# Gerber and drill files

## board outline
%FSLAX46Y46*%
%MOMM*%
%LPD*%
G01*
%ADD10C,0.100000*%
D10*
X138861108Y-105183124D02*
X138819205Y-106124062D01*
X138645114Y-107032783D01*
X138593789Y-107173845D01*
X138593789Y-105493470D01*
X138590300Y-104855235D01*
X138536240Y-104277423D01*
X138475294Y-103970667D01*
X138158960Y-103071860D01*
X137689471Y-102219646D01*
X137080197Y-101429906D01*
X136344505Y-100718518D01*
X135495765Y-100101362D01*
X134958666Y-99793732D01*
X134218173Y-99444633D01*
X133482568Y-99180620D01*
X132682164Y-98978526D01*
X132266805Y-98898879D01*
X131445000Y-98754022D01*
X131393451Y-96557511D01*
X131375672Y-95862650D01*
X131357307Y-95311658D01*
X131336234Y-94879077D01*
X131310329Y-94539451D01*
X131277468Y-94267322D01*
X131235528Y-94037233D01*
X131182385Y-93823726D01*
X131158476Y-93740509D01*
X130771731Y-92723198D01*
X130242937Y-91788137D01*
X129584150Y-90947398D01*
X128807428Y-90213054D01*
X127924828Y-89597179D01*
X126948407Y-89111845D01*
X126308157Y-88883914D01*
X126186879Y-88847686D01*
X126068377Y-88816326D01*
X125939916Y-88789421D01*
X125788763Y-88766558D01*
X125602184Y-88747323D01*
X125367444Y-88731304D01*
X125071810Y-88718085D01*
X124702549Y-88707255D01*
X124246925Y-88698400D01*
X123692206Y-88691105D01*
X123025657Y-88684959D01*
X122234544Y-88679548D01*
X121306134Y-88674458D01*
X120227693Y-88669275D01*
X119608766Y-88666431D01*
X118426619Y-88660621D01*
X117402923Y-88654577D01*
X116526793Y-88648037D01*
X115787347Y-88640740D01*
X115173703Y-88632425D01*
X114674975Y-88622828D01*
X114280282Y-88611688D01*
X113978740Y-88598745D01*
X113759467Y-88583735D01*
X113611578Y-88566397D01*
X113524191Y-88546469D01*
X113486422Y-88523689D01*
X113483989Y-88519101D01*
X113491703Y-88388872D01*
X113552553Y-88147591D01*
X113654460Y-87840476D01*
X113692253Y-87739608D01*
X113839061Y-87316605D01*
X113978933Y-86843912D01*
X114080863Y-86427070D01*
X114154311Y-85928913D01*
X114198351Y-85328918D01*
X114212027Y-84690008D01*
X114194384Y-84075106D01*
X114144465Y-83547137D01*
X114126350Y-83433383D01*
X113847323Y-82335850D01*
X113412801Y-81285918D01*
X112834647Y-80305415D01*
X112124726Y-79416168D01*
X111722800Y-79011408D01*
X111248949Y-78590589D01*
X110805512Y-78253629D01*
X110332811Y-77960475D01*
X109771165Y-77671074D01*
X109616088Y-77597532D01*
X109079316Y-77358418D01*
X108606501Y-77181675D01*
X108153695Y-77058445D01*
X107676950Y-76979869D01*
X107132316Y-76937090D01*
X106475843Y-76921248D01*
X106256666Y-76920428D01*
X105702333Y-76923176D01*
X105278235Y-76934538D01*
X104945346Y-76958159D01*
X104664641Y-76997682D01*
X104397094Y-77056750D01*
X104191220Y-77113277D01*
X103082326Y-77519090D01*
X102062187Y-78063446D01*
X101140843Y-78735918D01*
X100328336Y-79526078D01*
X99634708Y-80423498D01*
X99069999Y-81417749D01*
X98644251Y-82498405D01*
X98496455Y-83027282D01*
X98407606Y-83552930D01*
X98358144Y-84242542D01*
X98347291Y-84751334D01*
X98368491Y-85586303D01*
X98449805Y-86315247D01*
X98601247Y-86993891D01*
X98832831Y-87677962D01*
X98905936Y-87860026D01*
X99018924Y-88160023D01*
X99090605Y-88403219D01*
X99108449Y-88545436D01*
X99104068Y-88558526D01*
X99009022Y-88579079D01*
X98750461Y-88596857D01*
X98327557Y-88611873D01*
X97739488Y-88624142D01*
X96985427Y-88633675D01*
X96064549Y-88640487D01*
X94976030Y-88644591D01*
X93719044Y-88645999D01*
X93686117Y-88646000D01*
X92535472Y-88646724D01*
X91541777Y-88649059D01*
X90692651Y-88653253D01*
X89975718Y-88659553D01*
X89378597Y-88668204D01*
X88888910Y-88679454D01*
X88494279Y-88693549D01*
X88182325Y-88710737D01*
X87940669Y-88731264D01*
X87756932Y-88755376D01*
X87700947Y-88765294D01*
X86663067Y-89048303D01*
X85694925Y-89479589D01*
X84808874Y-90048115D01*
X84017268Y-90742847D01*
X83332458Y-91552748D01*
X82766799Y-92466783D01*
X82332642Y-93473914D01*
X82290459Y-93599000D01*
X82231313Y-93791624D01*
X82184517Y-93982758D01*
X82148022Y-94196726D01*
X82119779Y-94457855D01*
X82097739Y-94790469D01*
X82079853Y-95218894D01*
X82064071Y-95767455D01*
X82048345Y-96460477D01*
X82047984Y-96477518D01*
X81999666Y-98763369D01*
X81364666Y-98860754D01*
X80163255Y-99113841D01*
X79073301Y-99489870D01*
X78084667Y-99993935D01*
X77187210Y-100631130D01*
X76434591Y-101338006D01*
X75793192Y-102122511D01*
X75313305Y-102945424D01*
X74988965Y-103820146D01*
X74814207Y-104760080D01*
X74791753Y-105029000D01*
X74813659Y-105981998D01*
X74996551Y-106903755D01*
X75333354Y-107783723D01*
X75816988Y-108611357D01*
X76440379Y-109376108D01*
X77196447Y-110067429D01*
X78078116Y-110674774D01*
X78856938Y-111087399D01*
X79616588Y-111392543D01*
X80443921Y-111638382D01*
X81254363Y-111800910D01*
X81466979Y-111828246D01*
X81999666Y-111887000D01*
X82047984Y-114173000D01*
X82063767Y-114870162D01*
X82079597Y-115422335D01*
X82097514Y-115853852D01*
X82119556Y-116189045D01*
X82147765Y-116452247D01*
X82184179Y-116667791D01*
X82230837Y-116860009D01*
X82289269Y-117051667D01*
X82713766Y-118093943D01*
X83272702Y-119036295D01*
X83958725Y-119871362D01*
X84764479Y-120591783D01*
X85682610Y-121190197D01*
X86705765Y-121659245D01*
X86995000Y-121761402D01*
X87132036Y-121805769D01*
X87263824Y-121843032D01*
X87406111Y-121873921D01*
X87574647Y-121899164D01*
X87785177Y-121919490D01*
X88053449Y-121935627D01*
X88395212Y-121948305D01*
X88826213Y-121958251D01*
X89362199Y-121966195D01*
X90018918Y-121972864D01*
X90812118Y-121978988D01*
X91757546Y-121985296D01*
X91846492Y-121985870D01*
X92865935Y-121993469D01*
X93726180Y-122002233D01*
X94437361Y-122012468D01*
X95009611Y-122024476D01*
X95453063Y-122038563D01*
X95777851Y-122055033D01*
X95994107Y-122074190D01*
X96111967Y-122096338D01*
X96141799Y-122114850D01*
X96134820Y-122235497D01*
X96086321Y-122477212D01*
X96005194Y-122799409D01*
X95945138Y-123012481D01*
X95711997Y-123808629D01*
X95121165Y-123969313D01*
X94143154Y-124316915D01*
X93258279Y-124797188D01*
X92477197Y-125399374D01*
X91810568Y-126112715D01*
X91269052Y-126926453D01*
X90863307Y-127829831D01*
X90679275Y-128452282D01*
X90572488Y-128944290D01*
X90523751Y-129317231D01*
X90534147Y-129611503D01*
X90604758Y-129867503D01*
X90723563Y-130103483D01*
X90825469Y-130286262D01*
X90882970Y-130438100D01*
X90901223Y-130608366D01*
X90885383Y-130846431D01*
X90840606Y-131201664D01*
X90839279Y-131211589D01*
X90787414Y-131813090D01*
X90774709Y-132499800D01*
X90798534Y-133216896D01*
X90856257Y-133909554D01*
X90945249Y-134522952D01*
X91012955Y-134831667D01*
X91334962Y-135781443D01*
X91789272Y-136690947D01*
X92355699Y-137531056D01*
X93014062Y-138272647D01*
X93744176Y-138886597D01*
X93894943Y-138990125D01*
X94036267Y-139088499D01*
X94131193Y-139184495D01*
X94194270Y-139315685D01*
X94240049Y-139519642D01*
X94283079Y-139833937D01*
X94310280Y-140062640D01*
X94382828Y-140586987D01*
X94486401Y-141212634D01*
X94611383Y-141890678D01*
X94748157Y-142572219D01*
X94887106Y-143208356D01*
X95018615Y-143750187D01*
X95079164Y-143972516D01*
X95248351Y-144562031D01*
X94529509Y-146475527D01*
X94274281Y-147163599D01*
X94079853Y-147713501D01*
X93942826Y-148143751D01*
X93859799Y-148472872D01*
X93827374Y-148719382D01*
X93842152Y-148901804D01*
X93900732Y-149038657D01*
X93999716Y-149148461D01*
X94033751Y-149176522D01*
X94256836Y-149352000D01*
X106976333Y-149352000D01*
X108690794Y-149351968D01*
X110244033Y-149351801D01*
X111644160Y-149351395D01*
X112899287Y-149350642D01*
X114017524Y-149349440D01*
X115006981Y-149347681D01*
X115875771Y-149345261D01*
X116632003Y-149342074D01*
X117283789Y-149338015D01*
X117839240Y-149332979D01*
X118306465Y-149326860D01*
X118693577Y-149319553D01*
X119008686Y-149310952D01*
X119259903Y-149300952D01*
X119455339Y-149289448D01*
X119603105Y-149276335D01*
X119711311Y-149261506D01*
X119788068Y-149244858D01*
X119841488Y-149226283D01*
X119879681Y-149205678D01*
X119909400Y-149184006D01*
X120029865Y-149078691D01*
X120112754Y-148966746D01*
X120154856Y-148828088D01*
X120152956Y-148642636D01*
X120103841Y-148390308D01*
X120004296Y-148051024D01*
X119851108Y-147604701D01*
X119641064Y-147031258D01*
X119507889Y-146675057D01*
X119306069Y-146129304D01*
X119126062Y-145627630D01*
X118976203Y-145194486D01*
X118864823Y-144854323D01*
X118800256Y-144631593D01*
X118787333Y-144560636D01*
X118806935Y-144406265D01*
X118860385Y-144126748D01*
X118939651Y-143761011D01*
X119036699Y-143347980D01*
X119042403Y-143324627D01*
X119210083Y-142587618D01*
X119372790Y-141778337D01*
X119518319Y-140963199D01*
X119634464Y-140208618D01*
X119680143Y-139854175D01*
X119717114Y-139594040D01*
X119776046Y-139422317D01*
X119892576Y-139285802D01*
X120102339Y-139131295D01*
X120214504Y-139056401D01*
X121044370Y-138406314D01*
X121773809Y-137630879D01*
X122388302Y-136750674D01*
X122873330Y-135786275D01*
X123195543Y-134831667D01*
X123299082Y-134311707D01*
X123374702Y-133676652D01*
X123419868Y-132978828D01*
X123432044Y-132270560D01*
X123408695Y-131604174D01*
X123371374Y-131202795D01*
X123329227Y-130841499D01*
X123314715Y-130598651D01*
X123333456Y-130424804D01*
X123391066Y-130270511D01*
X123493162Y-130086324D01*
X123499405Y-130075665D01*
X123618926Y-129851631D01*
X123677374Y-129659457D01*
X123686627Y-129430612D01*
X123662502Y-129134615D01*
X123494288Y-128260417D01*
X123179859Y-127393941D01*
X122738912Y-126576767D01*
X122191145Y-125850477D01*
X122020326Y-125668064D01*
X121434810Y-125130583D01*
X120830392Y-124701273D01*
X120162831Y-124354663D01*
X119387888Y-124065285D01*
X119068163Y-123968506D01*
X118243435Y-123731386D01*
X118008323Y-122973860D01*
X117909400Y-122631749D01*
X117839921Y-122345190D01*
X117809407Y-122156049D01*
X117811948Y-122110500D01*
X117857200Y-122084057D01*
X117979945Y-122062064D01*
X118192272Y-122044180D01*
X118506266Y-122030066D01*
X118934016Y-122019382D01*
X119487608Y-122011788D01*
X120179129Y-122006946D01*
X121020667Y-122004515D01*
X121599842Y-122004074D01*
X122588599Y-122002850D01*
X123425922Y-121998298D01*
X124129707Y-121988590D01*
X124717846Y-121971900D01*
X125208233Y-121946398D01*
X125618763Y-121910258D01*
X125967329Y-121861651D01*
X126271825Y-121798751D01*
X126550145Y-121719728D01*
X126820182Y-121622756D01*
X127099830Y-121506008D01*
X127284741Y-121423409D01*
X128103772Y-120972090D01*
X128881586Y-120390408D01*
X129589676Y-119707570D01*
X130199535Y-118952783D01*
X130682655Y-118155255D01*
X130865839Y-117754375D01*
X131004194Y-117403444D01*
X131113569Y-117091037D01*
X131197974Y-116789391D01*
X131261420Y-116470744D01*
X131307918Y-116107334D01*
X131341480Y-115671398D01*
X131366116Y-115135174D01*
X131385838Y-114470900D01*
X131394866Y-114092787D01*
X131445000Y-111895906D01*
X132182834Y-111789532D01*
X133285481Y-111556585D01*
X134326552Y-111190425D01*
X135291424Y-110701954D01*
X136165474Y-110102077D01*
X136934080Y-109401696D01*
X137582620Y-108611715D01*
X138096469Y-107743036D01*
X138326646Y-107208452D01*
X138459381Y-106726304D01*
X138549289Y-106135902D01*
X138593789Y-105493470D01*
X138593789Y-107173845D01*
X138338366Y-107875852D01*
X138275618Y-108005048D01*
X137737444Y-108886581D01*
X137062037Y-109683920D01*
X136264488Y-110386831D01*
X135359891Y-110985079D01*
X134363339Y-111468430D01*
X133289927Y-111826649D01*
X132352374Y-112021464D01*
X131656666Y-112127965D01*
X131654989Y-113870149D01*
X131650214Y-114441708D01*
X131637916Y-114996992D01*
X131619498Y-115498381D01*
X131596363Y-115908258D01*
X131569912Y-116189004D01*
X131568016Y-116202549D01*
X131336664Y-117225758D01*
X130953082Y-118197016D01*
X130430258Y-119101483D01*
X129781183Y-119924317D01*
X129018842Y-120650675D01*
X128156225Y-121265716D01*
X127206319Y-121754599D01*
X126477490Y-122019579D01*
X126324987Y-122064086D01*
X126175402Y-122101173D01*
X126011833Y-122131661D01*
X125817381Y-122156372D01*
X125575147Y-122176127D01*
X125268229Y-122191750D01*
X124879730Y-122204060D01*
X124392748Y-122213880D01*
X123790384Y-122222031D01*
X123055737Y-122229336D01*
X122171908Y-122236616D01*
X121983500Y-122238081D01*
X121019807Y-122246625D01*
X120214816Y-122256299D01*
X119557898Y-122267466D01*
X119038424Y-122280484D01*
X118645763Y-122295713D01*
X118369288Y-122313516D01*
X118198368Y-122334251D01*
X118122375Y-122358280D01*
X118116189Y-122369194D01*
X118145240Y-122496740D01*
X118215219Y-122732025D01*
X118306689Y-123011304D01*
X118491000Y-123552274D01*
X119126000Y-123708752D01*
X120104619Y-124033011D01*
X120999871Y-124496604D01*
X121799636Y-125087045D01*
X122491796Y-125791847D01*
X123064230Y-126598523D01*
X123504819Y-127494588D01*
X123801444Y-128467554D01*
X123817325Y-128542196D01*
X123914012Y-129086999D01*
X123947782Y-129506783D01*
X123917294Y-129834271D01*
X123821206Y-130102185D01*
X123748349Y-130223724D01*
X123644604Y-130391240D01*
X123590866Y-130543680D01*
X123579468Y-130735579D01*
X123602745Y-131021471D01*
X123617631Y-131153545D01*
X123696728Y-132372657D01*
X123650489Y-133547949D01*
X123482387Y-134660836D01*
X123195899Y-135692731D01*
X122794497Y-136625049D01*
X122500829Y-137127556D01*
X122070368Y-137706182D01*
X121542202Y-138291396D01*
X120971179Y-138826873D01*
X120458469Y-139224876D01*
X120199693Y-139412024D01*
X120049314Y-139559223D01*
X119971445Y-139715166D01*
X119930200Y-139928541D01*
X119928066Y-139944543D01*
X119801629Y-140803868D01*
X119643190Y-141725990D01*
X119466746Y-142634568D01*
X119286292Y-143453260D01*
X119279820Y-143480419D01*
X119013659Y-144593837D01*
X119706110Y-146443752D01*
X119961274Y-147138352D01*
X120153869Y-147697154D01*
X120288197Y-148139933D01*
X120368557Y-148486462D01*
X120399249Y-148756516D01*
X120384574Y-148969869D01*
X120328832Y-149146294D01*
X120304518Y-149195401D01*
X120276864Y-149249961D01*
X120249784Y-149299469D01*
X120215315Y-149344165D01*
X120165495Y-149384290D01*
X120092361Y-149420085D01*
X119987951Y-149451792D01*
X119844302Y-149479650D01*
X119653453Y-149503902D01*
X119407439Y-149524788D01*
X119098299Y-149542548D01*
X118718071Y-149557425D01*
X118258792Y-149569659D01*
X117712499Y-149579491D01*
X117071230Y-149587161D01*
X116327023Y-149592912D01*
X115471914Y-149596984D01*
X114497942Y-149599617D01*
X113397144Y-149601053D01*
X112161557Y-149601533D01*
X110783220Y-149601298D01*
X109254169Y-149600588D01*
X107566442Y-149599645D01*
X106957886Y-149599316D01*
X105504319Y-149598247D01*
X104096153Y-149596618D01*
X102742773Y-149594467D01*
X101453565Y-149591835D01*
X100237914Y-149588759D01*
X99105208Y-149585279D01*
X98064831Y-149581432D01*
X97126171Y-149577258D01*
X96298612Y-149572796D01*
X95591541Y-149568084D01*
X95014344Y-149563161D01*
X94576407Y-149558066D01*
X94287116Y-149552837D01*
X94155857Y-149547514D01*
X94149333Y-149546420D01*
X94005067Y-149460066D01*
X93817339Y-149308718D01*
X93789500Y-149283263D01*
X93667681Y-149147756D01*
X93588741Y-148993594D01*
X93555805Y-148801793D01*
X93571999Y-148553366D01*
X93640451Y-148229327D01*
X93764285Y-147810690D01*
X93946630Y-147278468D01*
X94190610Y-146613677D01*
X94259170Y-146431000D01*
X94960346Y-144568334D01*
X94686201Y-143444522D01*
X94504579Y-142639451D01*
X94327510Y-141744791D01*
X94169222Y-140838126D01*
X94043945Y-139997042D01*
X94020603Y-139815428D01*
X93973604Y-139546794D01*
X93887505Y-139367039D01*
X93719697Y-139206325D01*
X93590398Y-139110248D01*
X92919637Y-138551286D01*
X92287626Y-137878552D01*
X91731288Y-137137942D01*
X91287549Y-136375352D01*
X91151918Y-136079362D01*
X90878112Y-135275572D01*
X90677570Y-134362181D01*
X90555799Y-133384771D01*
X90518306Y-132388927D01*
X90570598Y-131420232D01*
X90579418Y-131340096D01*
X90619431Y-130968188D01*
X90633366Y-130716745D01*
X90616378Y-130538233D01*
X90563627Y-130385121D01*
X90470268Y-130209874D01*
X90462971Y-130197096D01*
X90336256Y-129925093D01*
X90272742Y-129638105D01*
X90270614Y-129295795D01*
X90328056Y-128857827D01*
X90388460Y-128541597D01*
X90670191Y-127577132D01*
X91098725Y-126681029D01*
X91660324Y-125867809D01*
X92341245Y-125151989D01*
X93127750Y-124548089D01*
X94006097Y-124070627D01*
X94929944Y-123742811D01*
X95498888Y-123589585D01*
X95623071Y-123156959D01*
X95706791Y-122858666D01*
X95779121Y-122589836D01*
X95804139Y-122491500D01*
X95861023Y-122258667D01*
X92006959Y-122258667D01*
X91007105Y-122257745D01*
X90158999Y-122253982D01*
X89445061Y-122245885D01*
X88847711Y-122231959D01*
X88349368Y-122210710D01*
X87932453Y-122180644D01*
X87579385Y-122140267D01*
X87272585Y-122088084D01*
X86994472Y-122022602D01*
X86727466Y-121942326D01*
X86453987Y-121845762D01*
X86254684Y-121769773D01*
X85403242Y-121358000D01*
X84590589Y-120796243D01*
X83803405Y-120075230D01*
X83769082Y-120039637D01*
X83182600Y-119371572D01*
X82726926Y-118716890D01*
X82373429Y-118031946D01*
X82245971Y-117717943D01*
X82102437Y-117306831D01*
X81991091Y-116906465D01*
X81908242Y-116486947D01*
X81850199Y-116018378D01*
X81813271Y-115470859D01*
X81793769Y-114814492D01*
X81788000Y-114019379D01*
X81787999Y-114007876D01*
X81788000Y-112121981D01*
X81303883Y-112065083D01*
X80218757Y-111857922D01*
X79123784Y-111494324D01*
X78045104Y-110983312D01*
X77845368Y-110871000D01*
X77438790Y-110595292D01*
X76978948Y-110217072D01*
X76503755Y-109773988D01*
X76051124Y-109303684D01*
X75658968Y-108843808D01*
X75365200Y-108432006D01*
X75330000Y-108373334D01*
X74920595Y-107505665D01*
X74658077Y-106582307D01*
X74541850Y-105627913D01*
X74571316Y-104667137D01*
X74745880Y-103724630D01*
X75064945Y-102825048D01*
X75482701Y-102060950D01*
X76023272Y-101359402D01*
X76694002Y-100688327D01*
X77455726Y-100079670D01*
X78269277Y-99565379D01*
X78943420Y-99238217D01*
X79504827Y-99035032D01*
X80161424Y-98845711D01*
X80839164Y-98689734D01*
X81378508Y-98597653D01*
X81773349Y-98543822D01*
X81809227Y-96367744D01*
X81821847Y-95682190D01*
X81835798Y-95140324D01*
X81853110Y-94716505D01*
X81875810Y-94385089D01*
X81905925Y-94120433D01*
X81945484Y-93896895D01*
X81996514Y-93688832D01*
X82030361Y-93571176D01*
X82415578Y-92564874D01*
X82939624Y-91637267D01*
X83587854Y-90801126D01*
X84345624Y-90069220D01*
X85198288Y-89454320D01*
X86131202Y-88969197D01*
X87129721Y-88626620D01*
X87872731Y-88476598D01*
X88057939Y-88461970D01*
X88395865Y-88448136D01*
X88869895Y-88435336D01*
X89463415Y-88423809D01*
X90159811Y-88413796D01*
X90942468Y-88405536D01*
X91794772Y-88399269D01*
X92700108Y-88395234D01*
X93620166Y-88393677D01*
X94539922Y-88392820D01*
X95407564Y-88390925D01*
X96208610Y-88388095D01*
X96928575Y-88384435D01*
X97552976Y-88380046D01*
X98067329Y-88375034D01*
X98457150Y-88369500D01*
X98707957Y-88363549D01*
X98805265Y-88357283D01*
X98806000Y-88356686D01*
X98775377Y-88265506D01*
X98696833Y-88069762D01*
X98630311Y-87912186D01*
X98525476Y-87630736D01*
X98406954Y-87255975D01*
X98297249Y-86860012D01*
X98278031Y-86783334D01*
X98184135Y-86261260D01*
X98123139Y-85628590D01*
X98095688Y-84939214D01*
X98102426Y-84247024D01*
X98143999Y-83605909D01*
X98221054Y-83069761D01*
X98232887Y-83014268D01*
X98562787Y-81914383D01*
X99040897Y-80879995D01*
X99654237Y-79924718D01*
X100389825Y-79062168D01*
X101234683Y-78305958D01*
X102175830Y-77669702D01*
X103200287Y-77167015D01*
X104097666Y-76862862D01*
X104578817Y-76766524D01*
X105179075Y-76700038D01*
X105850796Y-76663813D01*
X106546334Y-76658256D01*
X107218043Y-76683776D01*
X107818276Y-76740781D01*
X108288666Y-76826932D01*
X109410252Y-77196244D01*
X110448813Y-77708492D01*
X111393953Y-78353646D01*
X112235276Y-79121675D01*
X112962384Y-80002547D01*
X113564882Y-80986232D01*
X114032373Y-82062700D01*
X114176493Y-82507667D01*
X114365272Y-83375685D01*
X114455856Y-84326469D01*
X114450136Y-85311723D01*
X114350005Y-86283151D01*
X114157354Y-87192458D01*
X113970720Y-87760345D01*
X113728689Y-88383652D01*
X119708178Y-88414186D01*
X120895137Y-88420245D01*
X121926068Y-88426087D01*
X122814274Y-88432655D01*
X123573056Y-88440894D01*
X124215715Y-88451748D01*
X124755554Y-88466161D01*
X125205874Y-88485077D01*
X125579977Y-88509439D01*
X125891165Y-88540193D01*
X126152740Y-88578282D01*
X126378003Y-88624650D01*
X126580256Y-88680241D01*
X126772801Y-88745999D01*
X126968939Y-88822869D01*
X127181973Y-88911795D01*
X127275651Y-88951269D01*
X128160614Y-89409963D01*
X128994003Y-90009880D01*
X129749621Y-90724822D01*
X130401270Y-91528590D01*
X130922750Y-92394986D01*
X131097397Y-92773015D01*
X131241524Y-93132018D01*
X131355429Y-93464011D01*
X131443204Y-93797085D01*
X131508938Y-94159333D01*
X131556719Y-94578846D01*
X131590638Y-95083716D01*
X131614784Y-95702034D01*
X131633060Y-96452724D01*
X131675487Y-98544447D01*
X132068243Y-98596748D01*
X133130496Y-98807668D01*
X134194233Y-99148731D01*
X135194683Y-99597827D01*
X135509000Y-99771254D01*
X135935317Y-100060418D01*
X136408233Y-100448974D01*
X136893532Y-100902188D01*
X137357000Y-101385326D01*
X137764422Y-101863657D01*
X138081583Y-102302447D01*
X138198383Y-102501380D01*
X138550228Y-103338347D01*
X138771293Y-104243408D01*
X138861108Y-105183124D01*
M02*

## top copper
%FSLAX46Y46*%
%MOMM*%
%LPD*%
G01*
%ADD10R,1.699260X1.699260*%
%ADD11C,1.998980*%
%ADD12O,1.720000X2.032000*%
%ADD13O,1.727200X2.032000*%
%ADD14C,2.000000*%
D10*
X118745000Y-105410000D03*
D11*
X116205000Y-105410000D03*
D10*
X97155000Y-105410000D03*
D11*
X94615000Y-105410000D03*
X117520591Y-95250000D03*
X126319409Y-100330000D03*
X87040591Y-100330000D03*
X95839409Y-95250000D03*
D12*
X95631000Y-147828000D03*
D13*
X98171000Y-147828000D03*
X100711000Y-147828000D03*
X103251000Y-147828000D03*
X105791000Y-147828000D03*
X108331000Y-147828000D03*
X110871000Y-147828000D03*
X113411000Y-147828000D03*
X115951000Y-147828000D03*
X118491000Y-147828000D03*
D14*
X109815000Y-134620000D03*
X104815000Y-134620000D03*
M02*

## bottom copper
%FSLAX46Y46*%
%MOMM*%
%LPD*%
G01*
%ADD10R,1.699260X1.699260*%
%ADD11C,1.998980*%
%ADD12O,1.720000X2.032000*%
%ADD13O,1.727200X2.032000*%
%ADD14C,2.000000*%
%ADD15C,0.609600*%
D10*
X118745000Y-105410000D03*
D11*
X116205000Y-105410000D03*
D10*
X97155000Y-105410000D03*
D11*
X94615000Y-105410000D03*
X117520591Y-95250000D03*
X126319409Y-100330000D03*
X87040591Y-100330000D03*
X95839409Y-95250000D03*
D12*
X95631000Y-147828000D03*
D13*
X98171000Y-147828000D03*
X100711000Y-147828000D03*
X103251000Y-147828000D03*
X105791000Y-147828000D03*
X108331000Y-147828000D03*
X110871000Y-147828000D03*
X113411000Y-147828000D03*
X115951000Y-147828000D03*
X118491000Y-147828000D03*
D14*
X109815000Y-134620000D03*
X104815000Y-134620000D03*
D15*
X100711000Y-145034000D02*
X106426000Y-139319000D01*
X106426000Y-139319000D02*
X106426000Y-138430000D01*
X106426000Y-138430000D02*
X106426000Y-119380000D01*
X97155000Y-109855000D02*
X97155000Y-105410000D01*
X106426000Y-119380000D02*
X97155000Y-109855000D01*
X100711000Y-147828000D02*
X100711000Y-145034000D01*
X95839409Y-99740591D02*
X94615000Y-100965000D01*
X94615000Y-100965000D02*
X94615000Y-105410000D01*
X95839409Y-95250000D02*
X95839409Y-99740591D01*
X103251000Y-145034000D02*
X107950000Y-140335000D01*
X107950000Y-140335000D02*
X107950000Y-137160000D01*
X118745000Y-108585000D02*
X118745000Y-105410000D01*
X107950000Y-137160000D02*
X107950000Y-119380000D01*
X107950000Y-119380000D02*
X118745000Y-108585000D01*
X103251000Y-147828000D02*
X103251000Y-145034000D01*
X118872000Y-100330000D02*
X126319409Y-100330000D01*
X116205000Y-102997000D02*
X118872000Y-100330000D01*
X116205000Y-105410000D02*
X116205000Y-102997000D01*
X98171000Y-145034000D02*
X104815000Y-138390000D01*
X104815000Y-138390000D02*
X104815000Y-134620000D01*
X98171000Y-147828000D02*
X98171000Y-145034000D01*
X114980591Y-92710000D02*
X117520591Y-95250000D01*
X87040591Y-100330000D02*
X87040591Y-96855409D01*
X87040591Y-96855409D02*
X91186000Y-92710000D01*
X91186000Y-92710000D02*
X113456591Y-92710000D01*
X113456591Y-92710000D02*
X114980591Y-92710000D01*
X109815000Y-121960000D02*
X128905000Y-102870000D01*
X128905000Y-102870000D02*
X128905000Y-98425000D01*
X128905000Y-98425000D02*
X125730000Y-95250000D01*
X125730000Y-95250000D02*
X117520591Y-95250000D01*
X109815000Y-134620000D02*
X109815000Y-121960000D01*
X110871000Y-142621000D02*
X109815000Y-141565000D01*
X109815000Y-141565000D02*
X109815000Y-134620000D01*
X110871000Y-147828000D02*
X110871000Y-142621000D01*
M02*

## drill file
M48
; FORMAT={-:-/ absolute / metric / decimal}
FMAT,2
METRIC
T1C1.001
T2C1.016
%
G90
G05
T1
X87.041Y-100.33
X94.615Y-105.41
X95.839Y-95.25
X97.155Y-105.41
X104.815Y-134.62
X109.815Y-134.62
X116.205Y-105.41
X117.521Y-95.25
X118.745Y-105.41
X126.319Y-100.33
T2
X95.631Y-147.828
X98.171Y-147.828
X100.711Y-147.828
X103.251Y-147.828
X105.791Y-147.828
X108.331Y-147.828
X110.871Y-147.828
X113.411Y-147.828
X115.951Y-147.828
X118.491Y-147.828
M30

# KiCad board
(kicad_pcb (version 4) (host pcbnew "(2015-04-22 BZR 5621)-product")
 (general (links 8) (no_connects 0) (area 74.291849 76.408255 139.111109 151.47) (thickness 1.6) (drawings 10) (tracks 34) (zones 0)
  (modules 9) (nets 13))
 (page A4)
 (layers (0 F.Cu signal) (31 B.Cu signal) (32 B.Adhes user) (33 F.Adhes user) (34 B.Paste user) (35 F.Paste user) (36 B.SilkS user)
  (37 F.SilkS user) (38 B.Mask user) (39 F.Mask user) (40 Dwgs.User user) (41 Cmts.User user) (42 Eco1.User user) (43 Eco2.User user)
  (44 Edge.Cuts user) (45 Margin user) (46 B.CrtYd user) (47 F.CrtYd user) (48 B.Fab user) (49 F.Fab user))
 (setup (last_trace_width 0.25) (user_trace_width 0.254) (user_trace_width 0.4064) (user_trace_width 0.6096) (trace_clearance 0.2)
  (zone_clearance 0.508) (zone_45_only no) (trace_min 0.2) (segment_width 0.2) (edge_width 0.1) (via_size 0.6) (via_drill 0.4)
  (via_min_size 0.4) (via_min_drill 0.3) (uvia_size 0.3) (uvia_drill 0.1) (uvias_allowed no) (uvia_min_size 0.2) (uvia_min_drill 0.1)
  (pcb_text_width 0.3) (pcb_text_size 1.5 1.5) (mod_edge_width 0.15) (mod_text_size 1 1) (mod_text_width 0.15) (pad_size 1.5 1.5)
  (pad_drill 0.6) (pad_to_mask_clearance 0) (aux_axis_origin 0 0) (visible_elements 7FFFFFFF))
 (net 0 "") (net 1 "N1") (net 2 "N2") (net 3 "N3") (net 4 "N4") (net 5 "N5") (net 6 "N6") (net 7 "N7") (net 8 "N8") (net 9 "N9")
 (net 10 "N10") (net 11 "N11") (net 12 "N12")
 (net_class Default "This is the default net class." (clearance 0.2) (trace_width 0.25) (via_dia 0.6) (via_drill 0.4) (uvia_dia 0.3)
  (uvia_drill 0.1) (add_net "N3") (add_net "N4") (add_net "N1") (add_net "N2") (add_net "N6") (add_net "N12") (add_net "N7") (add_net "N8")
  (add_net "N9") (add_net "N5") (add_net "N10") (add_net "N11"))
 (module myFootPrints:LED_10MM (layer F.Cu) (at 117.475 105.41 180)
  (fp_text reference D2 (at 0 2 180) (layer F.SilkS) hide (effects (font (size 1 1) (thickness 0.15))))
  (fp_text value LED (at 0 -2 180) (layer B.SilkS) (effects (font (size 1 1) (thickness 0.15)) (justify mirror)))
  (pad 1 thru_hole rect (at -1.27 0 270) (size 1.69926 1.69926) (drill 1.00076) (layers *.Cu *.Mask F.SilkS) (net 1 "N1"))
  (pad 2 thru_hole circle (at 1.27 0 180) (size 1.99898 1.99898) (drill 1.00076) (layers *.Cu *.Mask F.SilkS) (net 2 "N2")))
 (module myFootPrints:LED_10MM (layer F.Cu) (at 95.885 105.41 180)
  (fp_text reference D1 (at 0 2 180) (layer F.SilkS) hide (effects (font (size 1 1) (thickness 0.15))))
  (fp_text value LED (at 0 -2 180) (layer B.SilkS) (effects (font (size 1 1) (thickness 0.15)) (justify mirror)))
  (pad 1 thru_hole rect (at -1.27 0 270) (size 1.69926 1.69926) (drill 1.00076) (layers *.Cu *.Mask F.SilkS) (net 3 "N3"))
  (pad 2 thru_hole circle (at 1.27 0 180) (size 1.99898 1.99898) (drill 1.00076) (layers *.Cu *.Mask F.SilkS) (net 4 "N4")))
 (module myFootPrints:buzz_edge (layer F.Cu) (at 106.68 113.03)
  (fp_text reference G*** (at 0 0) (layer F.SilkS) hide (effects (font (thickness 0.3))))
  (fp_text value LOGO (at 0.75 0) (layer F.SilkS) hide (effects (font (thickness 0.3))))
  (fp_poly
   (pts (xy 32.181108 -7.846876) (xy 32.139205 -6.905938) (xy 31.965114 -5.997217) (xy 31.913789 -5.856155) (xy 31.913789 -7.53653)
    (xy 31.9103 -8.174765) (xy 31.85624 -8.752577) (xy 31.795294 -9.059333) (xy 31.47896 -9.95814) (xy 31.009471 -10.810354)
    (xy 30.400197 -11.600094) (xy 29.664505 -12.311482) (xy 28.815765 -12.928638) (xy 28.278666 -13.236268) (xy 27.538173 -13.585367)
    (xy 26.802568 -13.84938) (xy 26.002164 -14.051474) (xy 25.586805 -14.131121) (xy 24.765 -14.275978) (xy 24.713451 -16.472489)
    (xy 24.695672 -17.16735) (xy 24.677307 -17.718342) (xy 24.656234 -18.150923) (xy 24.630329 -18.490549) (xy 24.597468 -18.762678)
    (xy 24.555528 -18.992767) (xy 24.502385 -19.206274) (xy 24.478476 -19.289491) (xy 24.091731 -20.306802) (xy 23.562937 -21.241863)
    (xy 22.90415 -22.082602) (xy 22.127428 -22.816946) (xy 21.244828 -23.432821) (xy 20.268407 -23.918155) (xy 19.628157 -24.146086)
    (xy 19.506879 -24.182314) (xy 19.388377 -24.213674) (xy 19.259916 -24.240579) (xy 19.108763 -24.263442) (xy 18.922184 -24.282677)
    (xy 18.687444 -24.298696) (xy 18.39181 -24.311915) (xy 18.022549 -24.322745) (xy 17.566925 -24.3316) (xy 17.012206 -24.338895)
    (xy 16.345657 -24.345041) (xy 15.554544 -24.350452) (xy 14.626134 -24.355542) (xy 13.547693 -24.360725) (xy 12.928766 -24.363569)
    (xy 11.746619 -24.369379) (xy 10.722923 -24.375423) (xy 9.846793 -24.381963) (xy 9.107347 -24.38926) (xy 8.493703 -24.397575)
    (xy 7.994975 -24.407172) (xy 7.600282 -24.418312) (xy 7.29874 -24.431255) (xy 7.079467 -24.446265) (xy 6.931578 -24.463603)
    (xy 6.844191 -24.483531) (xy 6.806422 -24.506311) (xy 6.803989 -24.510899) (xy 6.811703 -24.641128) (xy 6.872553 -24.882409)
    (xy 6.97446 -25.189524) (xy 7.012253 -25.290392) (xy 7.159061 -25.713395) (xy 7.298933 -26.186088) (xy 7.400863 -26.60293)
    (xy 7.474311 -27.101087) (xy 7.518351 -27.701082) (xy 7.532027 -28.339992) (xy 7.514384 -28.954894) (xy 7.464465 -29.482863)
    (xy 7.44635 -29.596617) (xy 7.167323 -30.69415) (xy 6.732801 -31.744082) (xy 6.154647 -32.724585) (xy 5.444726 -33.613832)
    (xy 5.0428 -34.018592) (xy 4.568949 -34.439411) (xy 4.125512 -34.776371) (xy 3.652811 -35.069525) (xy 3.091165 -35.358926)
    (xy 2.936088 -35.432468) (xy 2.399316 -35.671582) (xy 1.926501 -35.848325) (xy 1.473695 -35.971555) (xy 0.99695 -36.050131)
    (xy 0.452316 -36.09291) (xy -0.204157 -36.108752) (xy -0.423334 -36.109572) (xy -0.977667 -36.106824) (xy -1.401765 -36.095462)
    (xy -1.734654 -36.071841) (xy -2.015359 -36.032318) (xy -2.282906 -35.97325) (xy -2.48878 -35.916723) (xy -3.597674 -35.51091)
    (xy -4.617813 -34.966554) (xy -5.539157 -34.294082) (xy -6.351664 -33.503922) (xy -7.045292 -32.606502) (xy -7.610001 -31.612251)
    (xy -8.035749 -30.531595) (xy -8.183545 -30.002718) (xy -8.272394 -29.47707) (xy -8.321856 -28.787458) (xy -8.332709 -28.278666)
    (xy -8.311509 -27.443697) (xy -8.230195 -26.714753) (xy -8.078753 -26.036109) (xy -7.847169 -25.352038) (xy -7.774064 -25.169974)
    (xy -7.661076 -24.869977) (xy -7.589395 -24.626781) (xy -7.571551 -24.484564) (xy -7.575932 -24.471474) (xy -7.670978 -24.450921)
    (xy -7.929539 -24.433143) (xy -8.352443 -24.418127) (xy -8.940512 -24.405858) (xy -9.694573 -24.396325) (xy -10.615451 -24.389513)
    (xy -11.70397 -24.385409) (xy -12.960956 -24.384001) (xy -12.993883 -24.384) (xy -14.144528 -24.383276) (xy -15.138223 -24.380941)
    (xy -15.987349 -24.376747) (xy -16.704282 -24.370447) (xy -17.301403 -24.361796) (xy -17.79109 -24.350546) (xy -18.185721 -24.336451)
    (xy -18.497675 -24.319263) (xy -18.739331 -24.298736) (xy -18.923068 -24.274624) (xy -18.979053 -24.264706) (xy -20.016933 -23.981697)
    (xy -20.985075 -23.550411) (xy -21.871126 -22.981885) (xy -22.662732 -22.287153) (xy -23.347542 -21.477252) (xy -23.913201 -20.563217)
    (xy -24.347358 -19.556086) (xy -24.389541 -19.431) (xy -24.448687 -19.238376) (xy -24.495483 -19.047242) (xy -24.531978 -18.833274)
    (xy -24.560221 -18.572145) (xy -24.582261 -18.239531) (xy -24.600147 -17.811106) (xy -24.615929 -17.262545) (xy -24.631655 -16.569523)
    (xy -24.632016 -16.552482) (xy -24.680334 -14.266631) (xy -25.315334 -14.169246) (xy -26.516745 -13.916159) (xy -27.606699 -13.54013)
    (xy -28.595333 -13.036065) (xy -29.49279 -12.39887) (xy -30.245409 -11.691994) (xy -30.886808 -10.907489) (xy -31.366695 -10.084576)
    (xy -31.691035 -9.209854) (xy -31.865793 -8.26992) (xy -31.888247 -8.001) (xy -31.866341 -7.048002) (xy -31.683449 -6.126245)
    (xy -31.346646 -5.246277) (xy -30.863012 -4.418643) (xy -30.239621 -3.653892) (xy -29.483553 -2.962571) (xy -28.601884 -2.355226)
    (xy -27.823062 -1.942601) (xy -27.063412 -1.637457) (xy -26.236079 -1.391618) (xy -25.425637 -1.22909) (xy -25.213021 -1.201754)
    (xy -24.680334 -1.143) (xy -24.632016 1.143) (xy -24.616233 1.840162) (xy -24.600403 2.392335) (xy -24.582486 2.823852)
    (xy -24.560444 3.159045) (xy -24.532235 3.422247) (xy -24.495821 3.637791) (xy -24.449163 3.830009) (xy -24.390731 4.021667)
    (xy -23.966234 5.063943) (xy -23.407298 6.006295) (xy -22.721275 6.841362) (xy -21.915521 7.561783) (xy -20.99739 8.160197)
    (xy -19.974235 8.629245) (xy -19.685 8.731402) (xy -19.547964 8.775769) (xy -19.416176 8.813032) (xy -19.273889 8.843921)
    (xy -19.105353 8.869164) (xy -18.894823 8.88949) (xy -18.626551 8.905627) (xy -18.284788 8.918305) (xy -17.853787 8.928251)
    (xy -17.317801 8.936195) (xy -16.661082 8.942864) (xy -15.867882 8.948988) (xy -14.922454 8.955296) (xy -14.833508 8.95587)
    (xy -13.814065 8.963469) (xy -12.95382 8.972233) (xy -12.242639 8.982468) (xy -11.670389 8.994476) (xy -11.226937 9.008563)
    (xy -10.902149 9.025033) (xy -10.685893 9.04419) (xy -10.568033 9.066338) (xy -10.538201 9.08485) (xy -10.54518 9.205497)
    (xy -10.593679 9.447212) (xy -10.674806 9.769409) (xy -10.734862 9.982481) (xy -10.968003 10.778629) (xy -11.558835 10.939313)
    (xy -12.536846 11.286915) (xy -13.421721 11.767188) (xy -14.202803 12.369374) (xy -14.869432 13.082715) (xy -15.410948 13.896453)
    (xy -15.816693 14.799831) (xy -16.000725 15.422282) (xy -16.107512 15.91429) (xy -16.156249 16.287231) (xy -16.145853 16.581503)
    (xy -16.075242 16.837503) (xy -15.956437 17.073483) (xy -15.854531 17.256262) (xy -15.79703 17.4081) (xy -15.778777 17.578366)
    (xy -15.794617 17.816431) (xy -15.839394 18.171664) (xy -15.840721 18.181589) (xy -15.892586 18.78309) (xy -15.905291 19.4698)
    (xy -15.881466 20.186896) (xy -15.823743 20.879554) (xy -15.734751 21.492952) (xy -15.667045 21.801667) (xy -15.345038 22.751443)
    (xy -14.890728 23.660947) (xy -14.324301 24.501056) (xy -13.665938 25.242647) (xy -12.935824 25.856597) (xy -12.785057 25.960125)
    (xy -12.643733 26.058499) (xy -12.548807 26.154495) (xy -12.48573 26.285685) (xy -12.439951 26.489642) (xy -12.396921 26.803937)
    (xy -12.36972 27.03264) (xy -12.297172 27.556987) (xy -12.193599 28.182634) (xy -12.068617 28.860678) (xy -11.931843 29.542219)
    (xy -11.792894 30.178356) (xy -11.661385 30.720187) (xy -11.600836 30.942516) (xy -11.431649 31.532031) (xy -12.150491 33.445527)
    (xy -12.405719 34.133599) (xy -12.600147 34.683501) (xy -12.737174 35.113751) (xy -12.820201 35.442872) (xy -12.852626 35.689382)
    (xy -12.837848 35.871804) (xy -12.779268 36.008657) (xy -12.680284 36.118461) (xy -12.646249 36.146522) (xy -12.423164 36.322)
    (xy 0.296333 36.322) (xy 2.010794 36.321968) (xy 3.564033 36.321801) (xy 4.96416 36.321395) (xy 6.219287 36.320642)
    (xy 7.337524 36.31944) (xy 8.326981 36.317681) (xy 9.195771 36.315261) (xy 9.952003 36.312074) (xy 10.603789 36.308015)
    (xy 11.15924 36.302979) (xy 11.626465 36.29686) (xy 12.013577 36.289553) (xy 12.328686 36.280952) (xy 12.579903 36.270952)
    (xy 12.775339 36.259448) (xy 12.923105 36.246335) (xy 13.031311 36.231506) (xy 13.108068 36.214858) (xy 13.161488 36.196283)
    (xy 13.199681 36.175678) (xy 13.2294 36.154006) (xy 13.349865 36.048691) (xy 13.432754 35.936746) (xy 13.474856 35.798088)
    (xy 13.472956 35.612636) (xy 13.423841 35.360308) (xy 13.324296 35.021024) (xy 13.171108 34.574701) (xy 12.961064 34.001258)
    (xy 12.827889 33.645057) (xy 12.626069 33.099304) (xy 12.446062 32.59763) (xy 12.296203 32.164486) (xy 12.184823 31.824323)
    (xy 12.120256 31.601593) (xy 12.107333 31.530636) (xy 12.126935 31.376265) (xy 12.180385 31.096748) (xy 12.259651 30.731011)
    (xy 12.356699 30.31798) (xy 12.362403 30.294627) (xy 12.530083 29.557618) (xy 12.69279 28.748337) (xy 12.838319 27.933199)
    (xy 12.954464 27.178618) (xy 13.000143 26.824175) (xy 13.037114 26.56404) (xy 13.096046 26.392317) (xy 13.212576 26.255802)
    (xy 13.422339 26.101295) (xy 13.534504 26.026401) (xy 14.36437 25.376314) (xy 15.093809 24.600879) (xy 15.708302 23.720674)
    (xy 16.19333 22.756275) (xy 16.515543 21.801667) (xy 16.619082 21.281707) (xy 16.694702 20.646652) (xy 16.739868 19.948828)
    (xy 16.752044 19.24056) (xy 16.728695 18.574174) (xy 16.691374 18.172795) (xy 16.649227 17.811499) (xy 16.634715 17.568651)
    (xy 16.653456 17.394804) (xy 16.711066 17.240511) (xy 16.813162 17.056324) (xy 16.819405 17.045665) (xy 16.938926 16.821631)
    (xy 16.997374 16.629457) (xy 17.006627 16.400612) (xy 16.982502 16.104615) (xy 16.814288 15.230417) (xy 16.499859 14.363941)
    (xy 16.058912 13.546767) (xy 15.511145 12.820477) (xy 15.340326 12.638064) (xy 14.75481 12.100583) (xy 14.150392 11.671273)
    (xy 13.482831 11.324663) (xy 12.707888 11.035285) (xy 12.388163 10.938506) (xy 11.563435 10.701386) (xy 11.328323 9.94386)
    (xy 11.2294 9.601749) (xy 11.159921 9.31519) (xy 11.129407 9.126049) (xy 11.131948 9.0805) (xy 11.1772 9.054057) (xy 11.299945 9.032064)
    (xy 11.512272 9.01418) (xy 11.826266 9.000066) (xy 12.254016 8.989382) (xy 12.807608 8.981788) (xy 13.499129 8.976946)
    (xy 14.340667 8.974515) (xy 14.919842 8.974074) (xy 15.908599 8.97285) (xy 16.745922 8.968298) (xy 17.449707 8.95859)
    (xy 18.037846 8.9419) (xy 18.528233 8.916398) (xy 18.938763 8.880258) (xy 19.287329 8.831651) (xy 19.591825 8.768751)
    (xy 19.870145 8.689728) (xy 20.140182 8.592756) (xy 20.41983 8.476008) (xy 20.604741 8.393409) (xy 21.423772 7.94209)
    (xy 22.201586 7.360408) (xy 22.909676 6.67757) (xy 23.519535 5.922783) (xy 24.002655 5.125255) (xy 24.185839 4.724375)
    (xy 24.324194 4.373444) (xy 24.433569 4.061037) (xy 24.517974 3.759391) (xy 24.58142 3.440744) (xy 24.627918 3.077334)
    (xy 24.66148 2.641398) (xy 24.686116 2.105174) (xy 24.705838 1.4409) (xy 24.714866 1.062787) (xy 24.765 -1.134094)
    (xy 25.502834 -1.240468) (xy 26.605481 -1.473415) (xy 27.646552 -1.839575) (xy 28.611424 -2.328046) (xy 29.485474 -2.927923)
    (xy 30.25408 -3.628304) (xy 30.90262 -4.418285) (xy 31.416469 -5.286964) (xy 31.646646 -5.821548) (xy 31.779381 -6.303696)
    (xy 31.869289 -6.894098) (xy 31.913789 -7.53653) (xy 31.913789 -5.856155) (xy 31.658366 -5.154148) (xy 31.595618 -5.024952)
    (xy 31.057444 -4.143419) (xy 30.382037 -3.34608) (xy 29.584488 -2.643169) (xy 28.679891 -2.044921) (xy 27.683339 -1.56157)
    (xy 26.609927 -1.203351) (xy 25.672374 -1.008536) (xy 24.976666 -0.902035) (xy 24.974989 0.840149) (xy 24.970214 1.411708)
    (xy 24.957916 1.966992) (xy 24.939498 2.468381) (xy 24.916363 2.878258) (xy 24.889912 3.159004) (xy 24.888016 3.172549)
    (xy 24.656664 4.195758) (xy 24.273082 5.167016) (xy 23.750258 6.071483) (xy 23.101183 6.894317) (xy 22.338842 7.620675)
    (xy 21.476225 8.235716) (xy 20.526319 8.724599) (xy 19.79749 8.989579) (xy 19.644987 9.034086) (xy 19.495402 9.071173)
    (xy 19.331833 9.101661) (xy 19.137381 9.126372) (xy 18.895147 9.146127) (xy 18.588229 9.16175) (xy 18.19973 9.17406)
    (xy 17.712748 9.18388) (xy 17.110384 9.192031) (xy 16.375737 9.199336) (xy 15.491908 9.206616) (xy 15.3035 9.208081)
    (xy 14.339807 9.216625) (xy 13.534816 9.226299) (xy 12.877898 9.237466) (xy 12.358424 9.250484) (xy 11.965763 9.265713)
    (xy 11.689288 9.283516) (xy 11.518368 9.304251) (xy 11.442375 9.32828) (xy 11.436189 9.339194) (xy 11.46524 9.46674)
    (xy 11.535219 9.702025) (xy 11.626689 9.981304) (xy 11.811 10.522274) (xy 12.446 10.678752) (xy 13.424619 11.003011)
    (xy 14.319871 11.466604) (xy 15.119636 12.057045) (xy 15.811796 12.761847) (xy 16.38423 13.568523) (xy 16.824819 14.464588)
    (xy 17.121444 15.437554) (xy 17.137325 15.512196) (xy 17.234012 16.056999) (xy 17.267782 16.476783) (xy 17.237294 16.804271)
    (xy 17.141206 17.072185) (xy 17.068349 17.193724) (xy 16.964604 17.36124) (xy 16.910866 17.51368) (xy 16.899468 17.705579)
    (xy 16.922745 17.991471) (xy 16.937631 18.123545) (xy 17.016728 19.342657) (xy 16.970489 20.517949) (xy 16.802387 21.630836)
    (xy 16.515899 22.662731) (xy 16.114497 23.595049) (xy 15.820829 24.097556) (xy 15.390368 24.676182) (xy 14.862202 25.261396)
    (xy 14.291179 25.796873) (xy 13.778469 26.194876) (xy 13.519693 26.382024) (xy 13.369314 26.529223) (xy 13.291445 26.685166)
    (xy 13.2502 26.898541) (xy 13.248066 26.914543) (xy 13.121629 27.773868) (xy 12.96319 28.69599) (xy 12.786746 29.604568)
    (xy 12.606292 30.42326) (xy 12.59982 30.450419) (xy 12.333659 31.563837) (xy 13.02611 33.413752) (xy 13.281274 34.108352)
    (xy 13.473869 34.667154) (xy 13.608197 35.109933) (xy 13.688557 35.456462) (xy 13.719249 35.726516) (xy 13.704574 35.939869)
    (xy 13.648832 36.116294) (xy 13.624518 36.165401) (xy 13.596864 36.219961) (xy 13.569784 36.269469) (xy 13.535315 36.314165)
    (xy 13.485495 36.35429) (xy 13.412361 36.390085) (xy 13.307951 36.421792) (xy 13.164302 36.44965) (xy 12.973453 36.473902)
    (xy 12.727439 36.494788) (xy 12.418299 36.512548) (xy 12.038071 36.527425) (xy 11.578792 36.539659) (xy 11.032499 36.549491)
    (xy 10.39123 36.557161) (xy 9.647023 36.562912) (xy 8.791914 36.566984) (xy 7.817942 36.569617) (xy 6.717144 36.571053)
    (xy 5.481557 36.571533) (xy 4.10322 36.571298) (xy 2.574169 36.570588) (xy 0.886442 36.569645) (xy 0.277886 36.569316)
    (xy -1.175681 36.568247) (xy -2.583847 36.566618) (xy -3.937227 36.564467) (xy -5.226435 36.561835) (xy -6.442086 36.558759)
    (xy -7.574792 36.555279) (xy -8.615169 36.551432) (xy -9.553829 36.547258) (xy -10.381388 36.542796) (xy -11.088459 36.538084)
    (xy -11.665656 36.533161) (xy -12.103593 36.528066) (xy -12.392884 36.522837) (xy -12.524143 36.517514) (xy -12.530667 36.51642)
    (xy -12.674933 36.430066) (xy -12.862661 36.278718) (xy -12.8905 36.253263) (xy -13.012319 36.117756) (xy -13.091259 35.963594)
    (xy -13.124195 35.771793) (xy -13.108001 35.523366) (xy -13.039549 35.199327) (xy -12.915715 34.78069) (xy -12.73337 34.248468)
    (xy -12.48939 33.583677) (xy -12.42083 33.401) (xy -11.719654 31.538334) (xy -11.993799 30.414522) (xy -12.175421 29.609451)
    (xy -12.35249 28.714791) (xy -12.510778 27.808126) (xy -12.636055 26.967042) (xy -12.659397 26.785428) (xy -12.706396 26.516794)
    (xy -12.792495 26.337039) (xy -12.960303 26.176325) (xy -13.089602 26.080248) (xy -13.760363 25.521286) (xy -14.392374 24.848552)
    (xy -14.948712 24.107942) (xy -15.392451 23.345352) (xy -15.528082 23.049362) (xy -15.801888 22.245572) (xy -16.00243 21.332181)
    (xy -16.124201 20.354771) (xy -16.161694 19.358927) (xy -16.109402 18.390232) (xy -16.100582 18.310096) (xy -16.060569 17.938188)
    (xy -16.046634 17.686745) (xy -16.063622 17.508233) (xy -16.116373 17.355121) (xy -16.209732 17.179874) (xy -16.217029 17.167096)
    (xy -16.343744 16.895093) (xy -16.407258 16.608105) (xy -16.409386 16.265795) (xy -16.351944 15.827827) (xy -16.29154 15.511597)
    (xy -16.009809 14.547132) (xy -15.581275 13.651029) (xy -15.019676 12.837809) (xy -14.338755 12.121989) (xy -13.55225 11.518089)
    (xy -12.673903 11.040627) (xy -11.750056 10.712811) (xy -11.181112 10.559585) (xy -11.056929 10.126959) (xy -10.973209 9.828666)
    (xy -10.900879 9.559836) (xy -10.875861 9.4615) (xy -10.818977 9.228667) (xy -14.673041 9.228667) (xy -15.672895 9.227745)
    (xy -16.521001 9.223982) (xy -17.234939 9.215885) (xy -17.832289 9.201959) (xy -18.330632 9.18071) (xy -18.747547 9.150644)
    (xy -19.100615 9.110267) (xy -19.407415 9.058084) (xy -19.685528 8.992602) (xy -19.952534 8.912326) (xy -20.226013 8.815762)
    (xy -20.425316 8.739773) (xy -21.276758 8.328) (xy -22.089411 7.766243) (xy -22.876595 7.04523) (xy -22.910918 7.009637)
    (xy -23.4974 6.341572) (xy -23.953074 5.68689) (xy -24.306571 5.001946) (xy -24.434029 4.687943) (xy -24.577563 4.276831)
    (xy -24.688909 3.876465) (xy -24.771758 3.456947) (xy -24.829801 2.988378) (xy -24.866729 2.440859) (xy -24.886231 1.784492)
    (xy -24.892 0.989379) (xy -24.892001 0.977876) (xy -24.892 -0.908019) (xy -25.376117 -0.964917) (xy -26.461243 -1.172078)
    (xy -27.556216 -1.535676) (xy -28.634896 -2.046688) (xy -28.834632 -2.159) (xy -29.24121 -2.434708) (xy -29.701052 -2.812928)
    (xy -30.176245 -3.256012) (xy -30.628876 -3.726316) (xy -31.021032 -4.186192) (xy -31.3148 -4.597994) (xy -31.35 -4.656666)
    (xy -31.759405 -5.524335) (xy -32.021923 -6.447693) (xy -32.13815 -7.402087) (xy -32.108684 -8.362863) (xy -31.93412 -9.30537)
    (xy -31.615055 -10.204952) (xy -31.197299 -10.96905) (xy -30.656728 -11.670598) (xy -29.985998 -12.341673) (xy -29.224274 -12.95033)
    (xy -28.410723 -13.464621) (xy -27.73658 -13.791783) (xy -27.175173 -13.994968) (xy -26.518576 -14.184289) (xy -25.840836 -14.340266)
    (xy -25.301492 -14.432347) (xy -24.906651 -14.486178) (xy -24.870773 -16.662256) (xy -24.858153 -17.34781) (xy -24.844202 -17.889676)
    (xy -24.82689 -18.313495) (xy -24.80419 -18.644911) (xy -24.774075 -18.909567) (xy -24.734516 -19.133105) (xy -24.683486 -19.341168)
    (xy -24.649639 -19.458824) (xy -24.264422 -20.465126) (xy -23.740376 -21.392733) (xy -23.092146 -22.228874) (xy -22.334376 -22.96078)
    (xy -21.481712 -23.57568) (xy -20.548798 -24.060803) (xy -19.550279 -24.40338) (xy -18.807269 -24.553402) (xy -18.622061 -24.56803)
    (xy -18.284135 -24.581864) (xy -17.810105 -24.594664) (xy -17.216585 -24.606191) (xy -16.520189 -24.616204) (xy -15.737532 -24.624464)
    (xy -14.885228 -24.630731) (xy -13.979892 -24.634766) (xy -13.059834 -24.636323) (xy -12.140078 -24.63718) (xy -11.272436 -24.639075)
    (xy -10.47139 -24.641905) (xy -9.751425 -24.645565) (xy -9.127024 -24.649954) (xy -8.612671 -24.654966) (xy -8.22285 -24.6605)
    (xy -7.972043 -24.666451) (xy -7.874735 -24.672717) (xy -7.874 -24.673314) (xy -7.904623 -24.764494) (xy -7.983167 -24.960238)
    (xy -8.049689 -25.117814) (xy -8.154524 -25.399264) (xy -8.273046 -25.774025) (xy -8.382751 -26.169988) (xy -8.401969 -26.246666)
    (xy -8.495865 -26.76874) (xy -8.556861 -27.40141) (xy -8.584312 -28.090786) (xy -8.577574 -28.782976) (xy -8.536001 -29.424091)
    (xy -8.458946 -29.960239) (xy -8.447113 -30.015732) (xy -8.117213 -31.115617) (xy -7.639103 -32.150005) (xy -7.025763 -33.105282)
    (xy -6.290175 -33.967832) (xy -5.445317 -34.724042) (xy -4.50417 -35.360298) (xy -3.479713 -35.862985) (xy -2.582334 -36.167138)
    (xy -2.101183 -36.263476) (xy -1.500925 -36.329962) (xy -0.829204 -36.366187) (xy -0.133666 -36.371744) (xy 0.538043 -36.346224)
    (xy 1.138276 -36.289219) (xy 1.608666 -36.203068) (xy 2.730252 -35.833756) (xy 3.768813 -35.321508) (xy 4.713953 -34.676354)
    (xy 5.555276 -33.908325) (xy 6.282384 -33.027453) (xy 6.884882 -32.043768) (xy 7.352373 -30.9673) (xy 7.496493 -30.522333)
    (xy 7.685272 -29.654315) (xy 7.775856 -28.703531) (xy 7.770136 -27.718277) (xy 7.670005 -26.746849) (xy 7.477354 -25.837542)
    (xy 7.29072 -25.269655) (xy 7.048689 -24.646348) (xy 13.028178 -24.615814) (xy 14.215137 -24.609755) (xy 15.246068 -24.603913)
    (xy 16.134274 -24.597345) (xy 16.893056 -24.589106) (xy 17.535715 -24.578252) (xy 18.075554 -24.563839) (xy 18.525874 -24.544923)
    (xy 18.899977 -24.520561) (xy 19.211165 -24.489807) (xy 19.47274 -24.451718) (xy 19.698003 -24.40535) (xy 19.900256 -24.349759)
    (xy 20.092801 -24.284001) (xy 20.288939 -24.207131) (xy 20.501973 -24.118205) (xy 20.595651 -24.078731) (xy 21.480614 -23.620037)
    (xy 22.314003 -23.02012) (xy 23.069621 -22.305178) (xy 23.72127 -21.50141) (xy 24.24275 -20.635014) (xy 24.417397 -20.256985)
    (xy 24.561524 -19.897982) (xy 24.675429 -19.565989) (xy 24.763204 -19.232915) (xy 24.828938 -18.870667) (xy 24.876719 -18.451154)
    (xy 24.910638 -17.946284) (xy 24.934784 -17.327966) (xy 24.95306 -16.577276) (xy 24.995487 -14.485553) (xy 25.388243 -14.433252)
    (xy 26.450496 -14.222332) (xy 27.514233 -13.881269) (xy 28.514683 -13.432173) (xy 28.829 -13.258746) (xy 29.255317 -12.969582)
    (xy 29.728233 -12.581026) (xy 30.213532 -12.127812) (xy 30.677 -11.644674) (xy 31.084422 -11.166343) (xy 31.401583 -10.727553)
    (xy 31.518383 -10.52862) (xy 31.870228 -9.691653) (xy 32.091293 -8.786592) (xy 32.181108 -7.846876) (xy 32.181108 -7.846876))
   (layer Edge.Cuts) (width 0.1)))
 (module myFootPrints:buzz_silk (layer F.Cu) (at 106.68 113.03)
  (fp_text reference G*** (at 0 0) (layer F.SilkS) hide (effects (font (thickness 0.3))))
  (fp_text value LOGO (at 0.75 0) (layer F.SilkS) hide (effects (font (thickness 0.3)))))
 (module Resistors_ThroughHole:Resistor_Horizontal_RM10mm (layer F.Cu) (at 121.92 97.79 330)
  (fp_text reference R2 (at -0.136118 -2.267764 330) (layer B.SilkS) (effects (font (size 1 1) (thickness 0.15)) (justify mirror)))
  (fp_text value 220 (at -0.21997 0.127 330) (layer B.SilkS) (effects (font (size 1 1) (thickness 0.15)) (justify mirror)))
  (pad 1 thru_hole circle (at -5.08 0 330) (size 1.99898 1.99898) (drill 1.00076) (layers *.Cu *.SilkS *.Mask) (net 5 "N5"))
  (pad 2 thru_hole circle (at 5.08 0 330) (size 1.99898 1.99898) (drill 1.00076) (layers *.Cu *.SilkS *.Mask) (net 2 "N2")))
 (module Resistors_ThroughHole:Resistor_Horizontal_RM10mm (layer F.Cu) (at 91.44 97.79 30)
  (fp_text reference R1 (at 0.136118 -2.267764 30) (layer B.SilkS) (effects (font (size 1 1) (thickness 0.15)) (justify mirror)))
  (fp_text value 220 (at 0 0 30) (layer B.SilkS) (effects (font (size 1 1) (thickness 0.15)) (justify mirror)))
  (pad 1 thru_hole circle (at -5.08 0 30) (size 1.99898 1.99898) (drill 1.00076) (layers *.Cu *.SilkS *.Mask) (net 5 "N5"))
  (pad 2 thru_hole circle (at 5.08 0 30) (size 1.99898 1.99898) (drill 1.00076) (layers *.Cu *.SilkS *.Mask) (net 4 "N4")))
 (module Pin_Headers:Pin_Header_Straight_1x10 (layer F.Cu) (at 95.631 147.828 90)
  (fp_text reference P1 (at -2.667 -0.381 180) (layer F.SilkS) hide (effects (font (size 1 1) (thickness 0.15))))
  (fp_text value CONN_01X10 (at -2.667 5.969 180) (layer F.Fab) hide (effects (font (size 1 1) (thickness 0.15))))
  (pad 1 thru_hole oval (at 0 0 90) (size 2.032 1.72) (drill 1.016) (layers *.Cu *.Mask F.SilkS) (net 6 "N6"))
  (pad 2 thru_hole oval (at 0 2.54 90) (size 2.032 1.7272) (drill 1.016) (layers *.Cu *.Mask F.SilkS) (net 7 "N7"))
  (pad 3 thru_hole oval (at 0 5.08 90) (size 2.032 1.7272) (drill 1.016) (layers *.Cu *.Mask F.SilkS) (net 3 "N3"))
  (pad 4 thru_hole oval (at 0 7.62 90) (size 2.032 1.7272) (drill 1.016) (layers *.Cu *.Mask F.SilkS) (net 1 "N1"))
  (pad 5 thru_hole oval (at 0 10.16 90) (size 2.032 1.7272) (drill 1.016) (layers *.Cu *.Mask F.SilkS) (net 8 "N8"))
  (pad 6 thru_hole oval (at 0 12.7 90) (size 2.032 1.7272) (drill 1.016) (layers *.Cu *.Mask F.SilkS) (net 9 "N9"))
  (pad 7 thru_hole oval (at 0 15.24 90) (size 2.032 1.7272) (drill 1.016) (layers *.Cu *.Mask F.SilkS) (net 5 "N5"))
  (pad 8 thru_hole oval (at 0 17.78 90) (size 2.032 1.7272) (drill 1.016) (layers *.Cu *.Mask F.SilkS) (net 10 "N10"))
  (pad 9 thru_hole oval (at 0 20.32 90) (size 2.032 1.7272) (drill 1.016) (layers *.Cu *.Mask F.SilkS) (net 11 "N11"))
  (pad 10 thru_hole oval (at 0 22.86 90) (size 2.032 1.7272) (drill 1.016) (layers *.Cu *.Mask F.SilkS) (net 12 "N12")))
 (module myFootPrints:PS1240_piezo (layer F.Cu) (at 107.315 134.62 180)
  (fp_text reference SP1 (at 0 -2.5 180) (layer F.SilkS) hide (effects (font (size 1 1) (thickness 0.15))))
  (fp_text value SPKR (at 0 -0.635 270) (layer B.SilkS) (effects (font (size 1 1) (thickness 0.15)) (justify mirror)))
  (pad 1 thru_hole circle (at -2.5 0 180) (size 2 2) (drill 1.00076) (layers *.Cu *.Mask F.SilkS) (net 5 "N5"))
  (pad 2 thru_hole circle (at 2.5 0 180) (size 2 2) (drill 1.00076) (layers *.Cu *.Mask F.SilkS) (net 7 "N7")))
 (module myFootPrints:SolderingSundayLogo (layer F.Cu) (at 106.045 100.33)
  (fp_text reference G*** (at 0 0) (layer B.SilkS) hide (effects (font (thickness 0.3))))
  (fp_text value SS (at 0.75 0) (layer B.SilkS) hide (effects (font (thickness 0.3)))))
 (segment (start 100.711 145.034) (end 106.426 139.319) (width 0.6096) (layer B.Cu) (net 3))
 (segment (start 106.426 139.319) (end 106.426 138.43) (width 0.6096) (layer B.Cu) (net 3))
 (segment (start 106.426 138.43) (end 106.426 119.38) (width 0.6096) (layer B.Cu) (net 3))
 (segment (start 97.155 109.855) (end 97.155 105.41) (width 0.6096) (layer B.Cu) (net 3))
 (segment (start 106.426 119.38) (end 97.155 109.855) (width 0.6096) (layer B.Cu) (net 3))
 (segment (start 100.711 147.828) (end 100.711 145.034) (width 0.6096) (layer B.Cu) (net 3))
 (segment (start 95.839409 99.740591) (end 94.615 100.965) (width 0.6096) (layer B.Cu) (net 4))
 (segment (start 94.615 100.965) (end 94.615 105.41) (width 0.6096) (layer B.Cu) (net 4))
 (segment (start 95.839409 95.25) (end 95.839409 99.740591) (width 0.6096) (layer B.Cu) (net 4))
 (segment (start 103.251 145.034) (end 107.95 140.335) (width 0.6096) (layer B.Cu) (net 1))
 (segment (start 107.95 140.335) (end 107.95 137.16) (width 0.6096) (layer B.Cu) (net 1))
 (segment (start 118.745 108.585) (end 118.745 105.41) (width 0.6096) (layer B.Cu) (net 1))
 (segment (start 107.95 137.16) (end 107.95 119.38) (width 0.6096) (layer B.Cu) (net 1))
 (segment (start 107.95 119.38) (end 118.745 108.585) (width 0.6096) (layer B.Cu) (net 1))
 (segment (start 103.251 147.828) (end 103.251 145.034) (width 0.6096) (layer B.Cu) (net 1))
 (segment (start 118.872 100.33) (end 126.319409 100.33) (width 0.6096) (layer B.Cu) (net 2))
 (segment (start 116.205 102.997) (end 118.872 100.33) (width 0.6096) (layer B.Cu) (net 2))
 (segment (start 116.205 105.41) (end 116.205 102.997) (width 0.6096) (layer B.Cu) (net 2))
 (segment (start 98.171 145.034) (end 104.815 138.39) (width 0.6096) (layer B.Cu) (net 7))
 (segment (start 104.815 138.39) (end 104.815 134.62) (width 0.6096) (layer B.Cu) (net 7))
 (segment (start 98.171 147.828) (end 98.171 145.034) (width 0.6096) (layer B.Cu) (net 7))
 (segment (start 114.980591 92.71) (end 117.520591 95.25) (width 0.6096) (layer B.Cu) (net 5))
 (segment (start 87.040591 100.33) (end 87.040591 96.855409) (width 0.6096) (layer B.Cu) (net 5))
 (segment (start 87.040591 96.855409) (end 91.186 92.71) (width 0.6096) (layer B.Cu) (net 5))
 (segment (start 91.186 92.71) (end 113.456591 92.71) (width 0.6096) (layer B.Cu) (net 5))
 (segment (start 113.456591 92.71) (end 114.980591 92.71) (width 0.6096) (layer B.Cu) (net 5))
 (segment (start 109.815 121.96) (end 128.905 102.87) (width 0.6096) (layer B.Cu) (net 5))
 (segment (start 128.905 102.87) (end 128.905 98.425) (width 0.6096) (layer B.Cu) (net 5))
 (segment (start 128.905 98.425) (end 125.73 95.25) (width 0.6096) (layer B.Cu) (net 5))
 (segment (start 125.73 95.25) (end 117.520591 95.25) (width 0.6096) (layer B.Cu) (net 5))
 (segment (start 109.815 134.62) (end 109.815 121.96) (width 0.6096) (layer B.Cu) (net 5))
 (segment (start 110.871 142.621) (end 109.815 141.565) (width 0.6096) (layer B.Cu) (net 5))
 (segment (start 109.815 141.565) (end 109.815 134.62) (width 0.6096) (layer B.Cu) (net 5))
 (segment (start 110.871 147.828) (end 110.871 142.621) (width 0.6096) (layer B.Cu) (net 5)))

